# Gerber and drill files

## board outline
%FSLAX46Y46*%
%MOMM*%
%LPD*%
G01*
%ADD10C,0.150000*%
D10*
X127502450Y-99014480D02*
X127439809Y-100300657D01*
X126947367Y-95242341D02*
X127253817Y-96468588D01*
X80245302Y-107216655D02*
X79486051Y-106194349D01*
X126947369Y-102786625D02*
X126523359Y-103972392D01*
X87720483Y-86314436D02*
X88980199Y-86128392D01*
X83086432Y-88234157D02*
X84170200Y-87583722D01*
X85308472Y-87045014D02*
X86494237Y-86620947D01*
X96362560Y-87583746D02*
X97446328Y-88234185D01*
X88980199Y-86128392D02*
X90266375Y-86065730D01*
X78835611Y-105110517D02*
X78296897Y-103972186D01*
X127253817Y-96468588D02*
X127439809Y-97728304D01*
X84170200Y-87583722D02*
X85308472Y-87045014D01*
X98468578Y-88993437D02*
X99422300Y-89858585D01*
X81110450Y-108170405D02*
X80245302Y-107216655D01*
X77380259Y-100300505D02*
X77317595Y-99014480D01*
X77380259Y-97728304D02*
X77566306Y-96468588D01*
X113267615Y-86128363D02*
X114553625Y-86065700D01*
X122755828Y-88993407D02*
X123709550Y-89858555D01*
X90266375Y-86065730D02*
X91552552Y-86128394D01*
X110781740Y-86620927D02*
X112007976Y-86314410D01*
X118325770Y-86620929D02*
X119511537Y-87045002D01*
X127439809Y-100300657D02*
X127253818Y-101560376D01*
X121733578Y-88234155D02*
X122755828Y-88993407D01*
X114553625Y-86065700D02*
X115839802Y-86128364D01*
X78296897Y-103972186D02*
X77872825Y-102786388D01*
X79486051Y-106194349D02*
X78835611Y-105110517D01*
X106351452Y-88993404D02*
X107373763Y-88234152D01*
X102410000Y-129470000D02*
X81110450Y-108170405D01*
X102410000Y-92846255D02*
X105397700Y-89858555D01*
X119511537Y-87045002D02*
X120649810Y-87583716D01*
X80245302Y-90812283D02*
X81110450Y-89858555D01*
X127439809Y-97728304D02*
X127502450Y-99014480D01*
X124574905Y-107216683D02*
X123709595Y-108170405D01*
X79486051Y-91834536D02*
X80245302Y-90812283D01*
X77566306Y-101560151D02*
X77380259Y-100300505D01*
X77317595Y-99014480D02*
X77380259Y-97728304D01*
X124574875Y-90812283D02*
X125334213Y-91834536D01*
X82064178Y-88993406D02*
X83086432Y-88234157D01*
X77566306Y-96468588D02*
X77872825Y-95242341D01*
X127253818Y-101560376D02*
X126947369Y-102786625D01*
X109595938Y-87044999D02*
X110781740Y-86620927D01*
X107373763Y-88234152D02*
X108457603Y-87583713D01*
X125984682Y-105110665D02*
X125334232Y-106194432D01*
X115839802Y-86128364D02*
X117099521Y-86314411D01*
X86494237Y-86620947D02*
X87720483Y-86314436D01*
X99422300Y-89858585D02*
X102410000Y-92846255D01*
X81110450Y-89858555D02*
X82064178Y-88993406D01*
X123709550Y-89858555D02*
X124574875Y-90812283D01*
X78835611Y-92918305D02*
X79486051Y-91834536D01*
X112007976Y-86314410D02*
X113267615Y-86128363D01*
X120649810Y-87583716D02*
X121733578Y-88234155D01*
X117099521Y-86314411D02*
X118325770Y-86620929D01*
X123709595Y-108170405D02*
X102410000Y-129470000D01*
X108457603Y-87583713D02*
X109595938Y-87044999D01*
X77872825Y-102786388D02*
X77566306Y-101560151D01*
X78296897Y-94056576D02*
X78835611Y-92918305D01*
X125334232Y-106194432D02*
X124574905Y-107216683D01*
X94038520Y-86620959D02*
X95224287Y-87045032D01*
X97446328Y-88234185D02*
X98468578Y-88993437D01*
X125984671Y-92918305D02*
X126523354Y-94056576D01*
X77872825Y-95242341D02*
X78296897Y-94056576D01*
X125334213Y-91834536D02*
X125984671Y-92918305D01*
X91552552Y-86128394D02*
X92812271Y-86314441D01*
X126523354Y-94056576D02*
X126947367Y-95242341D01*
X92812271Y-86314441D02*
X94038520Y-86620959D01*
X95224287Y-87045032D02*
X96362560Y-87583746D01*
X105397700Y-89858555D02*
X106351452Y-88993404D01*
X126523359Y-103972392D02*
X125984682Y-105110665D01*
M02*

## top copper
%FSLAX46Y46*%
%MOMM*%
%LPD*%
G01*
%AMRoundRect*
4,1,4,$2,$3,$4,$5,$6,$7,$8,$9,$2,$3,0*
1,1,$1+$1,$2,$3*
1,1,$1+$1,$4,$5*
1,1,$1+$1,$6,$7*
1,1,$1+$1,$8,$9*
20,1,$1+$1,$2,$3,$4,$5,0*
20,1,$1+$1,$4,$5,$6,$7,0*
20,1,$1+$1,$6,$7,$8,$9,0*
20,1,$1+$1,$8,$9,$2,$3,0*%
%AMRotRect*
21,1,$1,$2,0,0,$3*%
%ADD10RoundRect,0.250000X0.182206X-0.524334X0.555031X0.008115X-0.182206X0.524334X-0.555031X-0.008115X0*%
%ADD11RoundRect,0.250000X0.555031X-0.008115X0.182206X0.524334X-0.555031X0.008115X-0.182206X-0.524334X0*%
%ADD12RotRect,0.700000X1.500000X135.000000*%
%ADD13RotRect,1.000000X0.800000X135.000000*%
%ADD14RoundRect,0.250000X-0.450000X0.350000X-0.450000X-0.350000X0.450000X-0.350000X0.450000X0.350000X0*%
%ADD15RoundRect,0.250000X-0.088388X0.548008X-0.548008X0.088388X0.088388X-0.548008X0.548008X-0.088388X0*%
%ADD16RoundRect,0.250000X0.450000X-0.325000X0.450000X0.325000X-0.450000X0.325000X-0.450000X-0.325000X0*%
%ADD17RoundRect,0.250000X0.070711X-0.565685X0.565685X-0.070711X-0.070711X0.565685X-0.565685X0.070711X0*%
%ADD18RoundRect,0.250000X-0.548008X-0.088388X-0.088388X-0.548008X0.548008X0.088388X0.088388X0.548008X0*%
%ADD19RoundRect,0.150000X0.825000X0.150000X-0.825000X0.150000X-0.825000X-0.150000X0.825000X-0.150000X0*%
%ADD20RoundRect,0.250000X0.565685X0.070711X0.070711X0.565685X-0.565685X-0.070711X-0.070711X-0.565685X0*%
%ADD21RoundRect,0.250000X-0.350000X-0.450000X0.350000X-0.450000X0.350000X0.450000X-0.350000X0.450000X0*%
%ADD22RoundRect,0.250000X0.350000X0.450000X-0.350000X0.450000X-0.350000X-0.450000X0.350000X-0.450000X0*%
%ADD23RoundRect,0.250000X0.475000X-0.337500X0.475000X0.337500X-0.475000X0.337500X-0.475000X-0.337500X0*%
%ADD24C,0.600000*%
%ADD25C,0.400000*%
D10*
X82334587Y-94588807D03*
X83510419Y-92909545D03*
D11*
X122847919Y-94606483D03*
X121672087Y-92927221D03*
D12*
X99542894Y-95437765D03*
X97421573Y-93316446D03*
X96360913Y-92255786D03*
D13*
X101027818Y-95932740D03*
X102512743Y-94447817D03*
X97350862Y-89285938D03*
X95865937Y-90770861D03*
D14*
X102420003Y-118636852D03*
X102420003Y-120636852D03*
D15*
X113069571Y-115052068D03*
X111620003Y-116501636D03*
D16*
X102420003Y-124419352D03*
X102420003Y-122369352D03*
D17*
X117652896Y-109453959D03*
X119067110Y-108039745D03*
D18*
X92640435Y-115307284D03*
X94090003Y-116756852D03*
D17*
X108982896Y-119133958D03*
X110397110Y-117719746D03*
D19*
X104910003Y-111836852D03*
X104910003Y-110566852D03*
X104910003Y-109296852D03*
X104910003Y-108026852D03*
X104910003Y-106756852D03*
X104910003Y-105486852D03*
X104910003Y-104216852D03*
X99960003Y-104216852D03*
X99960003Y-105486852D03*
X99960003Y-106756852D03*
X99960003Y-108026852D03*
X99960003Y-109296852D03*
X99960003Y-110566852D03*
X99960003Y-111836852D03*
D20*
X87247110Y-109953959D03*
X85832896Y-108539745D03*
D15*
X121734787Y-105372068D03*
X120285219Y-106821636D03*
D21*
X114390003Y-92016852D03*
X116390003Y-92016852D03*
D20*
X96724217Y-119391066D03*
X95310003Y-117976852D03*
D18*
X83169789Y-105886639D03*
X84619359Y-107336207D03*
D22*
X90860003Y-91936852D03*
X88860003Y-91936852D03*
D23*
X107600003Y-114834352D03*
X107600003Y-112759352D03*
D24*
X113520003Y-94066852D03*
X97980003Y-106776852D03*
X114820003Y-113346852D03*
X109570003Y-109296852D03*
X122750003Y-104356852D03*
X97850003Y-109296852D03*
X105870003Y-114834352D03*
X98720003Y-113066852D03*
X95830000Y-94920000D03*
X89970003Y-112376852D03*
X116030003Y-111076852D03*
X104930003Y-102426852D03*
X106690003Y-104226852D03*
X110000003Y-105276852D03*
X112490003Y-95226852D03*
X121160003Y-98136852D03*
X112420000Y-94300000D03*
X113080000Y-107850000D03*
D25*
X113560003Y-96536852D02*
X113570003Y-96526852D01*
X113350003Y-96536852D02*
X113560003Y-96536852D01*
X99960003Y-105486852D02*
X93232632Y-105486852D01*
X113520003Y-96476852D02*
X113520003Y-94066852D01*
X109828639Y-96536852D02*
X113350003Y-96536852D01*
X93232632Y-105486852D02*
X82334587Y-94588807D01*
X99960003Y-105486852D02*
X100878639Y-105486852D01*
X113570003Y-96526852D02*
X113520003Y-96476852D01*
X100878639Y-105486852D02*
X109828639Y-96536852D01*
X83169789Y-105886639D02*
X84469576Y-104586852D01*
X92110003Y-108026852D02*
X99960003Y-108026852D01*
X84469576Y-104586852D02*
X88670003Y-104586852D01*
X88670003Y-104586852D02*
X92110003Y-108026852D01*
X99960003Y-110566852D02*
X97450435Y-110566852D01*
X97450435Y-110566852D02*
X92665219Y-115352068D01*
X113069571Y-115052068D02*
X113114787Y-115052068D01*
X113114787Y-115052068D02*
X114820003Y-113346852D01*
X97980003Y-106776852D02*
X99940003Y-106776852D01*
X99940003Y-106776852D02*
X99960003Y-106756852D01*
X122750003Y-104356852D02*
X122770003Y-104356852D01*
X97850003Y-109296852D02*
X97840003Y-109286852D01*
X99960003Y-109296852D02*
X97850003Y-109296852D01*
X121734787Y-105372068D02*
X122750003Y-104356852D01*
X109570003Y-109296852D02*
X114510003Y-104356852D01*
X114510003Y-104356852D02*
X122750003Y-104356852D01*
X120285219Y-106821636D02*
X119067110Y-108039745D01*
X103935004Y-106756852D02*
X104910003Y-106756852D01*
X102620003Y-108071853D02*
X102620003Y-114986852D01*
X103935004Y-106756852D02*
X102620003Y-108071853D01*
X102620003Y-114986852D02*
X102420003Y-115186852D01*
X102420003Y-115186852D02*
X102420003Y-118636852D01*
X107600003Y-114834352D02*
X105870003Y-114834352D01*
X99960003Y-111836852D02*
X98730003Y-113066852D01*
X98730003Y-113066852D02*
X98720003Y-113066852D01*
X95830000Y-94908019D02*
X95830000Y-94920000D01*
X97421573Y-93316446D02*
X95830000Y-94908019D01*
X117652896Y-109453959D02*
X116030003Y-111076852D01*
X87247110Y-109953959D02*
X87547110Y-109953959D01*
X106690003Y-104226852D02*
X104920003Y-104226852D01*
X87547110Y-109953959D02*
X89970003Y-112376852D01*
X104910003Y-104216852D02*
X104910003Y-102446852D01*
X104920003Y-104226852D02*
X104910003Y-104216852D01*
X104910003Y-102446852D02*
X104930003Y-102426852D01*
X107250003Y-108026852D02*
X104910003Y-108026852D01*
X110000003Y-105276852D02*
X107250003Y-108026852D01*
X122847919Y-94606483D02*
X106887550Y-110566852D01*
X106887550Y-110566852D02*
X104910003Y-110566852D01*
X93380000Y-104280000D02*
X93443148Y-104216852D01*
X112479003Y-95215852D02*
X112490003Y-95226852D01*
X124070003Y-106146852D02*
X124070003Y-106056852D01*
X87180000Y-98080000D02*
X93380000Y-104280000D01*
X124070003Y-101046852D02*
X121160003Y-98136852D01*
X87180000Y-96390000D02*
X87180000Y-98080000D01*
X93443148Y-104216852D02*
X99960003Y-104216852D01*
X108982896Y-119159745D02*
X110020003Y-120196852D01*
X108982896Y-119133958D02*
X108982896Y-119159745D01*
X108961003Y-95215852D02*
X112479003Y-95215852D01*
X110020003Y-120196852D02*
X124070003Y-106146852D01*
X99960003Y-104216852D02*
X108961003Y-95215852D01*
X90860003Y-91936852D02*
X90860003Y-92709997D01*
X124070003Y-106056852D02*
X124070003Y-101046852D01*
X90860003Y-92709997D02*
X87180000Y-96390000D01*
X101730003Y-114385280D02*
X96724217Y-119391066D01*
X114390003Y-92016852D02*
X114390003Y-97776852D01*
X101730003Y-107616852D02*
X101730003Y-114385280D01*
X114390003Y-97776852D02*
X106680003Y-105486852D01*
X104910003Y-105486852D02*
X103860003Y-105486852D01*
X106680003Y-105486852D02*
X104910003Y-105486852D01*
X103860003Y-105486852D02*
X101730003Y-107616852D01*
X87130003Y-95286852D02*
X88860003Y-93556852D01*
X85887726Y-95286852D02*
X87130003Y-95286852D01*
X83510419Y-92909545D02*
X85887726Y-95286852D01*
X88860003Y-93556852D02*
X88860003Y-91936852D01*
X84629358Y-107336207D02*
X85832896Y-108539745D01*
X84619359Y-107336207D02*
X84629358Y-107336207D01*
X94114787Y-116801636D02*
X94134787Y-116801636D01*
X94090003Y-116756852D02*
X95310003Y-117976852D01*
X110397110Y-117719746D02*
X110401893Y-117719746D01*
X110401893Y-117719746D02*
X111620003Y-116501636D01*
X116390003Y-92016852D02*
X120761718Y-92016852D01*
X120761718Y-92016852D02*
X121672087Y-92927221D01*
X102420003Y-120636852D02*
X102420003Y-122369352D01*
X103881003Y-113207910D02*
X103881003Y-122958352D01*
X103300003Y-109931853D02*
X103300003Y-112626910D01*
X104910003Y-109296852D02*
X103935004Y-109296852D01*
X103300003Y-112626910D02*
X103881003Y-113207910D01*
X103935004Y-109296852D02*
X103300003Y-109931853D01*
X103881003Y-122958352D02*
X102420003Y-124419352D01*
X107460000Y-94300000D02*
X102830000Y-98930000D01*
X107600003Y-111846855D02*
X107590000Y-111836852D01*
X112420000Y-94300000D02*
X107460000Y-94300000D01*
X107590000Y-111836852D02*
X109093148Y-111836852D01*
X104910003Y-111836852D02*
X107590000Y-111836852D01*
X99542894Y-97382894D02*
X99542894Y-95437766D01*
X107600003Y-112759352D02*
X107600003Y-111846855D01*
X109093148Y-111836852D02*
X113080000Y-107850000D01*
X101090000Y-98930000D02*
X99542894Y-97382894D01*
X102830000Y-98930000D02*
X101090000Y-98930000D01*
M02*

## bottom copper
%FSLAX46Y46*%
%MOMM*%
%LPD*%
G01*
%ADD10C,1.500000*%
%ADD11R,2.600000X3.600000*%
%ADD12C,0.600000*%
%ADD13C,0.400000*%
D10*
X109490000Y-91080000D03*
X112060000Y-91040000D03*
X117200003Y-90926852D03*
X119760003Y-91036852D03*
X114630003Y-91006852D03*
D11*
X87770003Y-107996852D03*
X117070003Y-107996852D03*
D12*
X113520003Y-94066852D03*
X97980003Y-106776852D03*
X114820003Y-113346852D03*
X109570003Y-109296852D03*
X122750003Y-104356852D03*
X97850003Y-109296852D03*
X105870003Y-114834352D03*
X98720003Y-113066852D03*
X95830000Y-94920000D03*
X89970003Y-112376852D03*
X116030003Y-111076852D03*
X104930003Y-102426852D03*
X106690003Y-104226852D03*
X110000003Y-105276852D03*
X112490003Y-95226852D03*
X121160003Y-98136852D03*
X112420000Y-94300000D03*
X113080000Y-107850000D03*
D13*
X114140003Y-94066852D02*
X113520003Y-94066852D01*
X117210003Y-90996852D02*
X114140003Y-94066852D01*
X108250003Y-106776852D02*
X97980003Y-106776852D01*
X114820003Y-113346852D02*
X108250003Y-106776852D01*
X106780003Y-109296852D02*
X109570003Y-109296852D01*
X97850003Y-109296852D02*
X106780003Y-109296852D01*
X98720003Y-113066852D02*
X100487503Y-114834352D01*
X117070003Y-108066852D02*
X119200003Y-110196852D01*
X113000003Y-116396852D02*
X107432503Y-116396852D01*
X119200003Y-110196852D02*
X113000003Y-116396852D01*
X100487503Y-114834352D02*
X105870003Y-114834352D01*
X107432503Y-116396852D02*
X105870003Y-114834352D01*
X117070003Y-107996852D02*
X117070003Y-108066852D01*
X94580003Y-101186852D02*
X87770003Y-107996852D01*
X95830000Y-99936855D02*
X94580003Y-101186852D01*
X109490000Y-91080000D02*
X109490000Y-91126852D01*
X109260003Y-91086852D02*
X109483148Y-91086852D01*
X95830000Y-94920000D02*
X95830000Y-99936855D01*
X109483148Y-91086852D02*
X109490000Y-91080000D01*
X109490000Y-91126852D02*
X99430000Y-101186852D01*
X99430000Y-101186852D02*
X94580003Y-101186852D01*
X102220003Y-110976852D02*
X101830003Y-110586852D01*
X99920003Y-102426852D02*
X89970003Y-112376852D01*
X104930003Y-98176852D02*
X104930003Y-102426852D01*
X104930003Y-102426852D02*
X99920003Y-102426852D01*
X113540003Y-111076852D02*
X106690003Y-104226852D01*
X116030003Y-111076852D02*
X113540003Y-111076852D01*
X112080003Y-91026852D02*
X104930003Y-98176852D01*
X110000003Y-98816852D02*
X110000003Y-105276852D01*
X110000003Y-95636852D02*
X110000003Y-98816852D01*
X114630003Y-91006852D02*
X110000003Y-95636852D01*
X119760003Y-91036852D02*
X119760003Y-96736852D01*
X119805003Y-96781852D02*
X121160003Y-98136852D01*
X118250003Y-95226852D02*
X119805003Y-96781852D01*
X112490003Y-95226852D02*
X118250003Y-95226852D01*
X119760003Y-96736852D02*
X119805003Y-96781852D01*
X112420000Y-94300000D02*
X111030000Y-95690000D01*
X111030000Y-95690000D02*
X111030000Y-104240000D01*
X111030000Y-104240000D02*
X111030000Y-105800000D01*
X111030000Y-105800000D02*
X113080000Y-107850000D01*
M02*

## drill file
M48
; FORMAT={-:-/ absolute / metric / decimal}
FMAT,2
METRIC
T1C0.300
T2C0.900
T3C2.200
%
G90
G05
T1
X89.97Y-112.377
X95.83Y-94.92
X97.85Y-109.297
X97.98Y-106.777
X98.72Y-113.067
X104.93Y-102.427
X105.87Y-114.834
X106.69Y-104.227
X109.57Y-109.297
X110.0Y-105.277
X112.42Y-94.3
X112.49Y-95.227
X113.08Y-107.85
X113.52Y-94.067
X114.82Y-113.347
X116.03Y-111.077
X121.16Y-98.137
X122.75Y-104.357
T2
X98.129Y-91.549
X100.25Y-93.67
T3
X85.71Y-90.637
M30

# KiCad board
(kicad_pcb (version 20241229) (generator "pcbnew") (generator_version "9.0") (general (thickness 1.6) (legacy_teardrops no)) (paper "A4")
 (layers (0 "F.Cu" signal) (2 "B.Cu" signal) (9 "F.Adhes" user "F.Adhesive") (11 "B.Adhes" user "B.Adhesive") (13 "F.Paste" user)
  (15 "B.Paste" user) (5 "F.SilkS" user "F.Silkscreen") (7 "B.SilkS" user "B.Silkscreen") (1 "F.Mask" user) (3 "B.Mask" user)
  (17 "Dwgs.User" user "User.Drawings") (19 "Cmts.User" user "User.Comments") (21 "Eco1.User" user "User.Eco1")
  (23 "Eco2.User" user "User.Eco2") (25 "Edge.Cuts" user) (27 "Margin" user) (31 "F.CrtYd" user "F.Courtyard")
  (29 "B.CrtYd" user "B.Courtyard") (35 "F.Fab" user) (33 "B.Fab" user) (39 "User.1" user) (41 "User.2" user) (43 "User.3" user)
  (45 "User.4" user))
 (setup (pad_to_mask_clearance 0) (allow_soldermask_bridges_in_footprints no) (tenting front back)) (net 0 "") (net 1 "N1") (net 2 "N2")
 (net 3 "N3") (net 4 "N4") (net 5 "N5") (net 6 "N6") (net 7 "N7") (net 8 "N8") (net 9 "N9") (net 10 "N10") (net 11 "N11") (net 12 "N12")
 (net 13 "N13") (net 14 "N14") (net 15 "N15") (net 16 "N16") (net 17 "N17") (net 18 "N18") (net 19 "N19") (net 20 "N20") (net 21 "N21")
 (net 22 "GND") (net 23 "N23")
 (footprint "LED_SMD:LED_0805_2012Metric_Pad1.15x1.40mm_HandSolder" (layer "F.Cu") (at 82.922503 93.749176 55)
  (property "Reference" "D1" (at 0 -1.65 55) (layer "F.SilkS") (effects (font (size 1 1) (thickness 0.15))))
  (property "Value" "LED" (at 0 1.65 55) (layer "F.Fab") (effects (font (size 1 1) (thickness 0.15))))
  (pad "1" smd roundrect (at -1.025 0 55) (size 1.15 1.4) (layers "F.Cu" "F.Mask" "F.Paste") (roundrect_rratio 0.217391) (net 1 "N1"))
  (pad "2" smd roundrect (at 1.025 0 55) (size 1.15 1.4) (layers "F.Cu" "F.Mask" "F.Paste") (roundrect_rratio 0.217391) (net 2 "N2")))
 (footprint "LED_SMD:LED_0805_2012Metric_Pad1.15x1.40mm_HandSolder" (layer "F.Cu") (at 122.260003 93.766852 125)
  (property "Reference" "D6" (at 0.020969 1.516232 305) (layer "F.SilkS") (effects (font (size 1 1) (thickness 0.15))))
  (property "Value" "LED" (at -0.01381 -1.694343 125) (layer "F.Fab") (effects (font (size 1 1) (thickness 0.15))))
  (pad "1" smd roundrect (at -1.025 0 125) (size 1.15 1.4) (layers "F.Cu" "F.Mask" "F.Paste") (roundrect_rratio 0.217391) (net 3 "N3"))
  (pad "2" smd roundrect (at 1.025 0 125) (size 1.15 1.4) (layers "F.Cu" "F.Mask" "F.Paste") (roundrect_rratio 0.217391) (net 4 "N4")))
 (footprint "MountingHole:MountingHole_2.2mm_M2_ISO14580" (layer "F.Cu") (at 85.710003 90.636852)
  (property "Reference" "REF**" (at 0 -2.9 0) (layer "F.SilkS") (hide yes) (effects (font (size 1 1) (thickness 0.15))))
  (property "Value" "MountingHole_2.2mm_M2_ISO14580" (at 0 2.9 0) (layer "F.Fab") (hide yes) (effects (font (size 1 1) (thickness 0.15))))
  (pad "" np_thru_hole circle (at 0 0) (size 2.2 2.2) (drill 2.2) (layers "*.Cu" "*.Mask")))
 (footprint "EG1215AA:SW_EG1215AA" (layer "F.Cu") (at 99.18934 92.609339 135)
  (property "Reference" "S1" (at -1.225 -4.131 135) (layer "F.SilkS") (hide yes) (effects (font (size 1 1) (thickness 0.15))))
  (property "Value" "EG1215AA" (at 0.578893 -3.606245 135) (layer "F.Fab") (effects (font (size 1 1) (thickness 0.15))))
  (pad "" np_thru_hole circle (at -1.5 -0.000001 135) (size 0.9 0.9) (drill 0.9) (layers "*.Cu" "*.Mask"))
  (pad "" np_thru_hole circle (at 1.5 0.000001 135) (size 0.9 0.9) (drill 0.9) (layers "*.Cu" "*.Mask"))
  (pad "1" smd rect (at -2.25 -1.749999 135) (size 0.7 1.5) (layers "F.Cu" "F.Mask" "F.Paste") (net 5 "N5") (solder_mask_margin 0.102))
  (pad "2" smd rect (at 0.75 -1.75 135) (size 0.7 1.5) (layers "F.Cu" "F.Mask" "F.Paste") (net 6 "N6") (solder_mask_margin 0.102))
  (pad "3" smd rect (at 2.25 -1.75 135) (size 0.7 1.5) (layers "F.Cu" "F.Mask" "F.Paste") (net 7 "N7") (solder_mask_margin 0.102))
  (pad "S1" smd rect (at -3.65 -1.049999 135) (size 1 0.8) (layers "F.Cu" "F.Mask" "F.Paste") (solder_mask_margin 0.102))
  (pad "S2" smd rect (at -3.650001 1.050001 135) (size 1 0.8) (layers "F.Cu" "F.Mask" "F.Paste") (solder_mask_margin 0.102))
  (pad "S3" smd rect (at 3.65 1.049999 135) (size 1 0.8) (layers "F.Cu" "F.Mask" "F.Paste") (solder_mask_margin 0.102))
  (pad "S4" smd rect (at 3.650001 -1.050001 135) (size 1 0.8) (layers "F.Cu" "F.Mask" "F.Paste") (solder_mask_margin 0.102)))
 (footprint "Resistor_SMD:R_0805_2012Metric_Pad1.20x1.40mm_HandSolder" (layer "F.Cu") (at 102.420003 119.636852 -90)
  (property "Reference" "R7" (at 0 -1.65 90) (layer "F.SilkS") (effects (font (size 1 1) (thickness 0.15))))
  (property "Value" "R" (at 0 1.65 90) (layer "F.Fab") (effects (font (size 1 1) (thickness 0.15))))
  (pad "1" smd roundrect (at -1 0 270) (size 1.2 1.4) (layers "F.Cu" "F.Mask" "F.Paste") (roundrect_rratio 0.208333) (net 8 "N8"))
  (pad "2" smd roundrect (at 1 0 270) (size 1.2 1.4) (layers "F.Cu" "F.Mask" "F.Paste") (roundrect_rratio 0.208333) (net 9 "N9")))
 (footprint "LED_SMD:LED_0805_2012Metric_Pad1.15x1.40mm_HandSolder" (layer "F.Cu") (at 112.344787 115.776852 -135)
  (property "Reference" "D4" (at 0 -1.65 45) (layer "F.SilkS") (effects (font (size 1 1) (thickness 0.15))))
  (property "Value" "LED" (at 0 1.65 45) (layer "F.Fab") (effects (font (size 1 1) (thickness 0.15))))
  (pad "1" smd roundrect (at -1.024999 0 225) (size 1.15 1.4) (layers "F.Cu" "F.Mask" "F.Paste") (roundrect_rratio 0.217391) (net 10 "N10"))
  (pad "2" smd roundrect (at 1.024999 0 225) (size 1.15 1.4) (layers "F.Cu" "F.Mask" "F.Paste") (roundrect_rratio 0.217391) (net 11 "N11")))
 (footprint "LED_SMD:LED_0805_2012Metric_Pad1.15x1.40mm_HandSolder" (layer "F.Cu") (at 102.420003 123.394352 90)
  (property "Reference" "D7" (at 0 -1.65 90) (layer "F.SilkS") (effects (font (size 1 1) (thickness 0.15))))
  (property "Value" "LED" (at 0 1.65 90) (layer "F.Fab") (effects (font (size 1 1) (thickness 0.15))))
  (pad "1" smd roundrect (at -1.025 0 90) (size 1.15 1.4) (layers "F.Cu" "F.Mask" "F.Paste") (roundrect_rratio 0.217391) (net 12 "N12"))
  (pad "2" smd roundrect (at 1.025 0 90) (size 1.15 1.4) (layers "F.Cu" "F.Mask" "F.Paste") (roundrect_rratio 0.217391) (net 9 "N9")))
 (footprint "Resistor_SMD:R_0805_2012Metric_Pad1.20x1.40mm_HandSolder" (layer "F.Cu") (at 118.360003 108.746852 45)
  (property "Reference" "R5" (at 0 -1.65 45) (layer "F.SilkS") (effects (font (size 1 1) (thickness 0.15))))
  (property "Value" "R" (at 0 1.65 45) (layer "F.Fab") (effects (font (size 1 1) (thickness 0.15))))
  (pad "1" smd roundrect (at -1 0 45) (size 1.2 1.4) (layers "F.Cu" "F.Mask" "F.Paste") (roundrect_rratio 0.208333) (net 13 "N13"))
  (pad "2" smd roundrect (at 1 0 45) (size 1.2 1.4) (layers "F.Cu" "F.Mask" "F.Paste") (roundrect_rratio 0.208333) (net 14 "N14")))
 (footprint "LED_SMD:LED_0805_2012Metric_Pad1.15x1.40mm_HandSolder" (layer "F.Cu") (at 93.365219 116.032068 -45)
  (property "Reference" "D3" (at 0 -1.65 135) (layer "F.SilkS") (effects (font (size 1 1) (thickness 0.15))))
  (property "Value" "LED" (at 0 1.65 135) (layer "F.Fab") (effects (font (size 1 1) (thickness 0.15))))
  (pad "1" smd roundrect (at -1.024999 0 315) (size 1.15 1.4) (layers "F.Cu" "F.Mask" "F.Paste") (roundrect_rratio 0.217391) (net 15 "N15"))
  (pad "2" smd roundrect (at 1.024999 0 315) (size 1.15 1.4) (layers "F.Cu" "F.Mask" "F.Paste") (roundrect_rratio 0.217391) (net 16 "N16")))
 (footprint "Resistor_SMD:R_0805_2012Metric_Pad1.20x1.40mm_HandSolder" (layer "F.Cu") (at 109.690003 118.426852 45)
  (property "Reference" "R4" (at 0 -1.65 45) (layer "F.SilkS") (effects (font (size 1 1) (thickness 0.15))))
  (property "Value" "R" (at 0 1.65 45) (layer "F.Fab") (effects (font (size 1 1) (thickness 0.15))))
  (pad "1" smd roundrect (at -1 -0.000001 45) (size 1.2 1.4) (layers "F.Cu" "F.Mask" "F.Paste") (roundrect_rratio 0.208333) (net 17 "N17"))
  (pad "2" smd roundrect (at 1 0.000001 45) (size 1.2 1.4) (layers "F.Cu" "F.Mask" "F.Paste") (roundrect_rratio 0.208333) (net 11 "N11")))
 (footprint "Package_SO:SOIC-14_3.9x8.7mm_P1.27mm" (layer "F.Cu") (at 102.435003 108.026852 180)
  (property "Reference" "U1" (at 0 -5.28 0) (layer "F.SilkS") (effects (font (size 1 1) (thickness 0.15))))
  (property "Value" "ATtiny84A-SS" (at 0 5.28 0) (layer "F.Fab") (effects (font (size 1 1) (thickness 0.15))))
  (pad "1" smd roundrect (at -2.475 -3.81 180) (size 1.95 0.6) (layers "F.Cu" "F.Mask" "F.Paste") (roundrect_rratio 0.25) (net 5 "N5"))
  (pad "2" smd roundrect (at -2.475 -2.54 180) (size 1.95 0.6) (layers "F.Cu" "F.Mask" "F.Paste") (roundrect_rratio 0.25) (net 3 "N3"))
  (pad "3" smd roundrect (at -2.475 -1.27 180) (size 1.95 0.6) (layers "F.Cu" "F.Mask" "F.Paste") (roundrect_rratio 0.25) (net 12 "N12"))
  (pad "4" smd roundrect (at -2.475 0 180) (size 1.95 0.6) (layers "F.Cu" "F.Mask" "F.Paste") (roundrect_rratio 0.25) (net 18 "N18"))
  (pad "5" smd roundrect (at -2.475 1.27 180) (size 1.95 0.6) (layers "F.Cu" "F.Mask" "F.Paste") (roundrect_rratio 0.25) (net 8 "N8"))
  (pad "6" smd roundrect (at -2.475 2.54 180) (size 1.95 0.6) (layers "F.Cu" "F.Mask" "F.Paste") (roundrect_rratio 0.25) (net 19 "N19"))
  (pad "7" smd roundrect (at -2.475 3.81 180) (size 1.95 0.6) (layers "F.Cu" "F.Mask" "F.Paste") (roundrect_rratio 0.25) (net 13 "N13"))
  (pad "8" smd roundrect (at 2.475 3.81 180) (size 1.95 0.6) (layers "F.Cu" "F.Mask" "F.Paste") (roundrect_rratio 0.25) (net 17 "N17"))
  (pad "9" smd roundrect (at 2.475 2.54 180) (size 1.95 0.6) (layers "F.Cu" "F.Mask" "F.Paste") (roundrect_rratio 0.25) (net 1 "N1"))
  (pad "10" smd roundrect (at 2.475 1.27 180) (size 1.95 0.6) (layers "F.Cu" "F.Mask" "F.Paste") (roundrect_rratio 0.25) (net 10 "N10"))
  (pad "11" smd roundrect (at 2.475 0 180) (size 1.95 0.6) (layers "F.Cu" "F.Mask" "F.Paste") (roundrect_rratio 0.25) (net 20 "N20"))
  (pad "12" smd roundrect (at 2.475 -1.27 180) (size 1.95 0.6) (layers "F.Cu" "F.Mask" "F.Paste") (roundrect_rratio 0.25) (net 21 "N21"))
  (pad "13" smd roundrect (at 2.475 -2.54 180) (size 1.95 0.6) (layers "F.Cu" "F.Mask" "F.Paste") (roundrect_rratio 0.25) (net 15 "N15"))
  (pad "14" smd roundrect (at 2.475 -3.81 180) (size 1.95 0.6) (layers "F.Cu" "F.Mask" "F.Paste") (roundrect_rratio 0.25) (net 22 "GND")))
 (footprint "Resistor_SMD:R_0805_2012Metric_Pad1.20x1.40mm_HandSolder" (layer "F.Cu") (at 86.540003 109.246852 135)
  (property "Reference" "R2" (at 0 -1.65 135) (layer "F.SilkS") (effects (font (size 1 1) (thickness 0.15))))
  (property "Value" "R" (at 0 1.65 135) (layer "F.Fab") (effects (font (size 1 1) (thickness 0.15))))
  (pad "1" smd roundrect (at -1 0 135) (size 1.2 1.4) (layers "F.Cu" "F.Mask" "F.Paste") (roundrect_rratio 0.208333) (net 13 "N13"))
  (pad "2" smd roundrect (at 1 0 135) (size 1.2 1.4) (layers "F.Cu" "F.Mask" "F.Paste") (roundrect_rratio 0.208333) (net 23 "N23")))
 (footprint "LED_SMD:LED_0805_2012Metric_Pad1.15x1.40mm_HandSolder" (layer "F.Cu") (at 121.010003 106.096852 -135)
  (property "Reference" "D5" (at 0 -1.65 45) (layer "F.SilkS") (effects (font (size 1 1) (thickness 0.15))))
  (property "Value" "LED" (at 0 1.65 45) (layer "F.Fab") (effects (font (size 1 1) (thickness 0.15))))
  (pad "1" smd roundrect (at -1.024999 0 225) (size 1.15 1.4) (layers "F.Cu" "F.Mask" "F.Paste") (roundrect_rratio 0.217391) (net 21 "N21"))
  (pad "2" smd roundrect (at 1.024999 0 225) (size 1.15 1.4) (layers "F.Cu" "F.Mask" "F.Paste") (roundrect_rratio 0.217391) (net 14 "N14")))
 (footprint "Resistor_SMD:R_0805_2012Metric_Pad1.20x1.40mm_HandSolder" (layer "F.Cu") (at 115.390003 92.016852)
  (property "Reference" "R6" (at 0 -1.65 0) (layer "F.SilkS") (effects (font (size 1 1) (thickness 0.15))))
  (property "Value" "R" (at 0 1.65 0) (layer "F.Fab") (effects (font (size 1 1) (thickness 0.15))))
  (pad "1" smd roundrect (at -1 0) (size 1.2 1.4) (layers "F.Cu" "F.Mask" "F.Paste") (roundrect_rratio 0.208333) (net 19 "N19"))
  (pad "2" smd roundrect (at 1 0) (size 1.2 1.4) (layers "F.Cu" "F.Mask" "F.Paste") (roundrect_rratio 0.208333) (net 4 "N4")))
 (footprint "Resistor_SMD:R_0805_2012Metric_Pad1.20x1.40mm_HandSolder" (layer "F.Cu") (at 96.01711 118.683959 135)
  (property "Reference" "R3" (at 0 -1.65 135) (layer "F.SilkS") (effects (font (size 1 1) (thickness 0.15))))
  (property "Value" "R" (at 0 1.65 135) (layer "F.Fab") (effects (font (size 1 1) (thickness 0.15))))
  (pad "1" smd roundrect (at -1 0 135) (size 1.2 1.4) (layers "F.Cu" "F.Mask" "F.Paste") (roundrect_rratio 0.208333) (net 19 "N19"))
  (pad "2" smd roundrect (at 1 0 135) (size 1.2 1.4) (layers "F.Cu" "F.Mask" "F.Paste") (roundrect_rratio 0.208333) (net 16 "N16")))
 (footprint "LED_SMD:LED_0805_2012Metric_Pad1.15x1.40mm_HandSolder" (layer "F.Cu") (at 83.894574 106.611423 -45)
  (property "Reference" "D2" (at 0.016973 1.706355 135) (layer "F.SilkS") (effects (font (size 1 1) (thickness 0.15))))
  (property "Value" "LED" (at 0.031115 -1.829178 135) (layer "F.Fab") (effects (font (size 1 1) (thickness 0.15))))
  (pad "1" smd roundrect (at -1.025 0.000001 315) (size 1.15 1.4) (layers "F.Cu" "F.Mask" "F.Paste") (roundrect_rratio 0.217391)
   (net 20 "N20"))
  (pad "2" smd roundrect (at 1.025 -0.000001 315) (size 1.15 1.4) (layers "F.Cu" "F.Mask" "F.Paste") (roundrect_rratio 0.217391)
   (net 23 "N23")))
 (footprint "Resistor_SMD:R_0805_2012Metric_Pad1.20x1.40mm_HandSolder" (layer "F.Cu") (at 89.860003 91.936852 180)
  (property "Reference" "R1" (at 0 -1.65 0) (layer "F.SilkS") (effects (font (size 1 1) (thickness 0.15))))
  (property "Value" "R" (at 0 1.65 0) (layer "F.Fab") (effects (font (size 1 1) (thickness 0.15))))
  (pad "1" smd roundrect (at -1 0 180) (size 1.2 1.4) (layers "F.Cu" "F.Mask" "F.Paste") (roundrect_rratio 0.208333) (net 17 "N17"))
  (pad "2" smd roundrect (at 1 0 180) (size 1.2 1.4) (layers "F.Cu" "F.Mask" "F.Paste") (roundrect_rratio 0.208333) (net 2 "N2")))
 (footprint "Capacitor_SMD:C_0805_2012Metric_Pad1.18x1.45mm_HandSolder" (layer "F.Cu") (at 107.600003 113.796852 90)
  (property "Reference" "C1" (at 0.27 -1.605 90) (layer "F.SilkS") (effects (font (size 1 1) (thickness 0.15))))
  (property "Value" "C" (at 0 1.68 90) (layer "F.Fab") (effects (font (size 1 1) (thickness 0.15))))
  (pad "1" smd roundrect (at -1.0375 0 90) (size 1.175 1.45) (layers "F.Cu" "F.Mask" "F.Paste") (roundrect_rratio 0.212766) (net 22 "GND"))
  (pad "2" smd roundrect (at 1.0375 0 90) (size 1.175 1.45) (layers "F.Cu" "F.Mask" "F.Paste") (roundrect_rratio 0.212766) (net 5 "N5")))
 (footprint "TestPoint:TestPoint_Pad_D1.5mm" (layer "B.Cu") (at 109.49 91.08)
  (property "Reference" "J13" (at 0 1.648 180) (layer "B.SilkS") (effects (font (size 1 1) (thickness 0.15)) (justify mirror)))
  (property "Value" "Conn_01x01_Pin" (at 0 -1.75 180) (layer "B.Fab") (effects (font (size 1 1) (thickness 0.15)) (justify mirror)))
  (pad "1" smd circle (at 0 0) (size 1.5 1.5) (layers "B.Cu" "B.Mask") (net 6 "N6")))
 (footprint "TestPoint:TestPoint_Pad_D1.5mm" (layer "B.Cu") (at 112.06 91.04)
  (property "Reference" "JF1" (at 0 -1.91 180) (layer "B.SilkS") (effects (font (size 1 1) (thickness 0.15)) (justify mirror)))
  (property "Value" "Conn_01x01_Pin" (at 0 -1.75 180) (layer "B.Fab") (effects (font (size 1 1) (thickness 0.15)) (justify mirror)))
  (pad "1" smd circle (at 0 0) (size 1.5 1.5) (layers "B.Cu" "B.Mask") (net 13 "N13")))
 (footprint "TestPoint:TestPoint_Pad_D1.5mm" (layer "B.Cu") (at 117.200003 90.926852)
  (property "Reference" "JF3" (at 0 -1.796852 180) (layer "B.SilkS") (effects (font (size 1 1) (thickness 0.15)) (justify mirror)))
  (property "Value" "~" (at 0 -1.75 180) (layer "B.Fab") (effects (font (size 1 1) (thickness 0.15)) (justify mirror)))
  (pad "1" smd circle (at 0 0) (size 1.5 1.5) (layers "B.Cu" "B.Mask") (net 1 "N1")))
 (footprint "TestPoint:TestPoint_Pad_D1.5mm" (layer "B.Cu") (at 119.760003 91.036852)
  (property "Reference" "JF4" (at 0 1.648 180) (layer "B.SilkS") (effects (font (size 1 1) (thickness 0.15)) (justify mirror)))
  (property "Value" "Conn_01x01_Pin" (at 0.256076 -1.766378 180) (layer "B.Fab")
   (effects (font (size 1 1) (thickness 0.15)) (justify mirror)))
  (pad "1" smd circle (at 0 0) (size 1.5 1.5) (layers "B.Cu" "B.Mask") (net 17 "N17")))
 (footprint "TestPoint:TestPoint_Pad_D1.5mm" (layer "B.Cu") (at 114.630003 91.006852)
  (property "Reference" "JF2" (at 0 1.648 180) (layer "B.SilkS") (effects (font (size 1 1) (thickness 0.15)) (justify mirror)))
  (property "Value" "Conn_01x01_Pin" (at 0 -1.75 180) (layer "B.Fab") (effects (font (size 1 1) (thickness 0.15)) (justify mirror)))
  (pad "1" smd circle (at 0 0) (size 1.5 1.5) (layers "B.Cu" "B.Mask") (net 18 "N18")))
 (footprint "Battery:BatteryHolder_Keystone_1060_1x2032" (layer "B.Cu") (at 102.420003 107.996852)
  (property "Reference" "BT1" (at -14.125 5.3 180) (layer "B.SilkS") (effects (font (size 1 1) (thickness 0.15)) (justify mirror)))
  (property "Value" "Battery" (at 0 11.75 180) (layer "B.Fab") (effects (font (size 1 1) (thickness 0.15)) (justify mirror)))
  (pad "1" smd rect (at -14.65 0 180) (size 2.6 3.6) (layers "B.Cu" "B.Mask" "B.Paste") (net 6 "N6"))
  (pad "2" smd rect (at 14.65 0 180) (size 2.6 3.6) (layers "B.Cu" "B.Mask" "B.Paste") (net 22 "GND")))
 (gr_line (start 127.50245 99.01448) (end 127.439809 100.300657) (stroke (width 0.15) (type default)) (layer "Edge.Cuts"))
 (gr_line (start 126.947367 95.242341) (end 127.253817 96.468588) (stroke (width 0.15) (type default)) (layer "Edge.Cuts"))
 (gr_line (start 80.245302 107.216655) (end 79.486051 106.194349) (stroke (width 0.15) (type default)) (layer "Edge.Cuts"))
 (gr_line (start 126.947369 102.786625) (end 126.523359 103.972392) (stroke (width 0.15) (type default)) (layer "Edge.Cuts"))
 (gr_line (start 87.720483 86.314436) (end 88.980199 86.128392) (stroke (width 0.15) (type default)) (layer "Edge.Cuts"))
 (gr_line (start 83.086432 88.234157) (end 84.1702 87.583722) (stroke (width 0.15) (type default)) (layer "Edge.Cuts"))
 (gr_line (start 85.308472 87.045014) (end 86.494237 86.620947) (stroke (width 0.15) (type default)) (layer "Edge.Cuts"))
 (gr_line (start 96.36256 87.583746) (end 97.446328 88.234185) (stroke (width 0.15) (type default)) (layer "Edge.Cuts"))
 (gr_line (start 88.980199 86.128392) (end 90.266375 86.06573) (stroke (width 0.15) (type default)) (layer "Edge.Cuts"))
 (gr_line (start 78.835611 105.110517) (end 78.296897 103.972186) (stroke (width 0.15) (type default)) (layer "Edge.Cuts"))
 (gr_line (start 127.253817 96.468588) (end 127.439809 97.728304) (stroke (width 0.15) (type default)) (layer "Edge.Cuts"))
 (gr_line (start 84.1702 87.583722) (end 85.308472 87.045014) (stroke (width 0.15) (type default)) (layer "Edge.Cuts"))
 (gr_line (start 98.468578 88.993437) (end 99.4223 89.858585) (stroke (width 0.15) (type default)) (layer "Edge.Cuts"))
 (gr_line (start 81.11045 108.170405) (end 80.245302 107.216655) (stroke (width 0.15) (type default)) (layer "Edge.Cuts"))
 (gr_line (start 77.380259 100.300505) (end 77.317595 99.01448) (stroke (width 0.15) (type default)) (layer "Edge.Cuts"))
 (gr_line (start 77.380259 97.728304) (end 77.566306 96.468588) (stroke (width 0.15) (type default)) (layer "Edge.Cuts"))
 (gr_line (start 113.267615 86.128363) (end 114.553625 86.0657) (stroke (width 0.15) (type default)) (layer "Edge.Cuts"))
 (gr_line (start 122.755828 88.993407) (end 123.70955 89.858555) (stroke (width 0.15) (type default)) (layer "Edge.Cuts"))
 (gr_line (start 90.266375 86.06573) (end 91.552552 86.128394) (stroke (width 0.15) (type default)) (layer "Edge.Cuts"))
 (gr_line (start 110.78174 86.620927) (end 112.007976 86.31441) (stroke (width 0.15) (type default)) (layer "Edge.Cuts"))
 (gr_line (start 118.32577 86.620929) (end 119.511537 87.045002) (stroke (width 0.15) (type default)) (layer "Edge.Cuts"))
 (gr_line (start 127.439809 100.300657) (end 127.253818 101.560376) (stroke (width 0.15) (type default)) (layer "Edge.Cuts"))
 (gr_line (start 121.733578 88.234155) (end 122.755828 88.993407) (stroke (width 0.15) (type default)) (layer "Edge.Cuts"))
 (gr_line (start 114.553625 86.0657) (end 115.839802 86.128364) (stroke (width 0.15) (type default)) (layer "Edge.Cuts"))
 (gr_line (start 78.296897 103.972186) (end 77.872825 102.786388) (stroke (width 0.15) (type default)) (layer "Edge.Cuts"))
 (gr_line (start 79.486051 106.194349) (end 78.835611 105.110517) (stroke (width 0.15) (type default)) (layer "Edge.Cuts"))
 (gr_line (start 106.351452 88.993404) (end 107.373763 88.234152) (stroke (width 0.15) (type default)) (layer "Edge.Cuts"))
 (gr_line (start 102.41 129.47) (end 81.11045 108.170405) (stroke (width 0.15) (type default)) (layer "Edge.Cuts"))
 (gr_line (start 102.41 92.846255) (end 105.3977 89.858555) (stroke (width 0.15) (type default)) (layer "Edge.Cuts"))
 (gr_line (start 119.511537 87.045002) (end 120.64981 87.583716) (stroke (width 0.15) (type default)) (layer "Edge.Cuts"))
 (gr_line (start 80.245302 90.812283) (end 81.11045 89.858555) (stroke (width 0.15) (type default)) (layer "Edge.Cuts"))
 (gr_line (start 127.439809 97.728304) (end 127.50245 99.01448) (stroke (width 0.15) (type default)) (layer "Edge.Cuts"))
 (gr_line (start 124.574905 107.216683) (end 123.709595 108.170405) (stroke (width 0.15) (type default)) (layer "Edge.Cuts"))
 (gr_line (start 79.486051 91.834536) (end 80.245302 90.812283) (stroke (width 0.15) (type default)) (layer "Edge.Cuts"))
 (gr_line (start 77.566306 101.560151) (end 77.380259 100.300505) (stroke (width 0.15) (type default)) (layer "Edge.Cuts"))
 (gr_line (start 77.317595 99.01448) (end 77.380259 97.728304) (stroke (width 0.15) (type default)) (layer "Edge.Cuts"))
 (gr_line (start 124.574875 90.812283) (end 125.334213 91.834536) (stroke (width 0.15) (type default)) (layer "Edge.Cuts"))
 (gr_line (start 82.064178 88.993406) (end 83.086432 88.234157) (stroke (width 0.15) (type default)) (layer "Edge.Cuts"))
 (gr_line (start 77.566306 96.468588) (end 77.872825 95.242341) (stroke (width 0.15) (type default)) (layer "Edge.Cuts"))
 (gr_line (start 127.253818 101.560376) (end 126.947369 102.786625) (stroke (width 0.15) (type default)) (layer "Edge.Cuts"))
 (gr_line (start 109.595938 87.044999) (end 110.78174 86.620927) (stroke (width 0.15) (type default)) (layer "Edge.Cuts"))
 (gr_line (start 107.373763 88.234152) (end 108.457603 87.583713) (stroke (width 0.15) (type default)) (layer "Edge.Cuts"))
 (gr_line (start 125.984682 105.110665) (end 125.334232 106.194432) (stroke (width 0.15) (type default)) (layer "Edge.Cuts"))
 (gr_line (start 115.839802 86.128364) (end 117.099521 86.314411) (stroke (width 0.15) (type default)) (layer "Edge.Cuts"))
 (gr_line (start 86.494237 86.620947) (end 87.720483 86.314436) (stroke (width 0.15) (type default)) (layer "Edge.Cuts"))
 (gr_line (start 99.4223 89.858585) (end 102.41 92.846255) (stroke (width 0.15) (type default)) (layer "Edge.Cuts"))
 (gr_line (start 81.11045 89.858555) (end 82.064178 88.993406) (stroke (width 0.15) (type default)) (layer "Edge.Cuts"))
 (gr_line (start 123.70955 89.858555) (end 124.574875 90.812283) (stroke (width 0.15) (type default)) (layer "Edge.Cuts"))
 (gr_line (start 78.835611 92.918305) (end 79.486051 91.834536) (stroke (width 0.15) (type default)) (layer "Edge.Cuts"))
 (gr_line (start 112.007976 86.31441) (end 113.267615 86.128363) (stroke (width 0.15) (type default)) (layer "Edge.Cuts"))
 (gr_line (start 120.64981 87.583716) (end 121.733578 88.234155) (stroke (width 0.15) (type default)) (layer "Edge.Cuts"))
 (gr_line (start 117.099521 86.314411) (end 118.32577 86.620929) (stroke (width 0.15) (type default)) (layer "Edge.Cuts"))
 (gr_line (start 123.709595 108.170405) (end 102.41 129.47) (stroke (width 0.15) (type default)) (layer "Edge.Cuts"))
 (gr_line (start 108.457603 87.583713) (end 109.595938 87.044999) (stroke (width 0.15) (type default)) (layer "Edge.Cuts"))
 (gr_line (start 77.872825 102.786388) (end 77.566306 101.560151) (stroke (width 0.15) (type default)) (layer "Edge.Cuts"))
 (gr_line (start 78.296897 94.056576) (end 78.835611 92.918305) (stroke (width 0.15) (type default)) (layer "Edge.Cuts"))
 (gr_line (start 125.334232 106.194432) (end 124.574905 107.216683) (stroke (width 0.15) (type default)) (layer "Edge.Cuts"))
 (gr_line (start 94.03852 86.620959) (end 95.224287 87.045032) (stroke (width 0.15) (type default)) (layer "Edge.Cuts"))
 (gr_line (start 97.446328 88.234185) (end 98.468578 88.993437) (stroke (width 0.15) (type default)) (layer "Edge.Cuts"))
 (gr_line (start 125.984671 92.918305) (end 126.523354 94.056576) (stroke (width 0.15) (type default)) (layer "Edge.Cuts"))
 (gr_line (start 77.872825 95.242341) (end 78.296897 94.056576) (stroke (width 0.15) (type default)) (layer "Edge.Cuts"))
 (gr_line (start 125.334213 91.834536) (end 125.984671 92.918305) (stroke (width 0.15) (type default)) (layer "Edge.Cuts"))
 (gr_line (start 91.552552 86.128394) (end 92.812271 86.314441) (stroke (width 0.15) (type default)) (layer "Edge.Cuts"))
 (gr_line (start 126.523354 94.056576) (end 126.947367 95.242341) (stroke (width 0.15) (type default)) (layer "Edge.Cuts"))
 (gr_line (start 92.812271 86.314441) (end 94.03852 86.620959) (stroke (width 0.15) (type default)) (layer "Edge.Cuts"))
 (gr_line (start 95.224287 87.045032) (end 96.36256 87.583746) (stroke (width 0.15) (type default)) (layer "Edge.Cuts"))
 (gr_line (start 105.3977 89.858555) (end 106.351452 88.993404) (stroke (width 0.15) (type default)) (layer "Edge.Cuts"))
 (gr_line (start 126.523359 103.972392) (end 125.984682 105.110665) (stroke (width 0.15) (type default)) (layer "Edge.Cuts"))
 (segment (start 113.560003 96.536852) (end 113.570003 96.526852) (width 0.4) (layer "F.Cu") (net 1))
 (segment (start 113.350003 96.536852) (end 113.560003 96.536852) (width 0.4) (layer "F.Cu") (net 1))
 (segment (start 99.960003 105.486852) (end 93.232632 105.486852) (width 0.4) (layer "F.Cu") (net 1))
 (segment (start 113.520003 96.476852) (end 113.520003 94.066852) (width 0.4) (layer "F.Cu") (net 1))
 (segment (start 109.828639 96.536852) (end 113.350003 96.536852) (width 0.4) (layer "F.Cu") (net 1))
 (segment (start 93.232632 105.486852) (end 82.334587 94.588807) (width 0.4) (layer "F.Cu") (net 1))
 (segment (start 99.960003 105.486852) (end 100.878639 105.486852) (width 0.4) (layer "F.Cu") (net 1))
 (segment (start 113.570003 96.526852) (end 113.520003 96.476852) (width 0.4) (layer "F.Cu") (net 1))
 (segment (start 100.878639 105.486852) (end 109.828639 96.536852) (width 0.4) (layer "F.Cu") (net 1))
 (via (at 113.520003 94.066852) (size 0.6) (drill 0.3) (layers "F.Cu" "B.Cu") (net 1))
 (segment (start 114.140003 94.066852) (end 113.520003 94.066852) (width 0.4) (layer "B.Cu") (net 1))
 (segment (start 117.210003 90.996852) (end 114.140003 94.066852) (width 0.4) (layer "B.Cu") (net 1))
 (segment (start 83.169789 105.886639) (end 84.469576 104.586852) (width 0.4) (layer "F.Cu") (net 20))
 (segment (start 92.110003 108.026852) (end 99.960003 108.026852) (width 0.4) (layer "F.Cu") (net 20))
 (segment (start 84.469576 104.586852) (end 88.670003 104.586852) (width 0.4) (layer "F.Cu") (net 20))
 (segment (start 88.670003 104.586852) (end 92.110003 108.026852) (width 0.4) (layer "F.Cu") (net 20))
 (segment (start 99.960003 110.566852) (end 97.450435 110.566852) (width 0.4) (layer "F.Cu") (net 15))
 (segment (start 97.450435 110.566852) (end 92.665219 115.352068) (width 0.4) (layer "F.Cu") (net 15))
 (segment (start 113.069571 115.052068) (end 113.114787 115.052068) (width 0.4) (layer "F.Cu") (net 10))
 (segment (start 113.114787 115.052068) (end 114.820003 113.346852) (width 0.4) (layer "F.Cu") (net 10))
 (segment (start 97.980003 106.776852) (end 99.940003 106.776852) (width 0.4) (layer "F.Cu") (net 10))
 (segment (start 99.940003 106.776852) (end 99.960003 106.756852) (width 0.4) (layer "F.Cu") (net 10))
 (via (at 97.980003 106.776852) (size 0.6) (drill 0.3) (layers "F.Cu" "B.Cu") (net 10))
 (via (at 114.820003 113.346852) (size 0.6) (drill 0.3) (layers "F.Cu" "B.Cu") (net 10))
 (segment (start 108.250003 106.776852) (end 97.980003 106.776852) (width 0.4) (layer "B.Cu") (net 10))
 (segment (start 114.820003 113.346852) (end 108.250003 106.776852) (width 0.4) (layer "B.Cu") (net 10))
 (segment (start 122.750003 104.356852) (end 122.770003 104.356852) (width 0.4) (layer "F.Cu") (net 21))
 (segment (start 97.850003 109.296852) (end 97.840003 109.286852) (width 0.4) (layer "F.Cu") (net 21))
 (segment (start 99.960003 109.296852) (end 97.850003 109.296852) (width 0.4) (layer "F.Cu") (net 21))
 (segment (start 121.734787 105.372068) (end 122.750003 104.356852) (width 0.4) (layer "F.Cu") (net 21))
 (segment (start 109.570003 109.296852) (end 114.510003 104.356852) (width 0.4) (layer "F.Cu") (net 21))
 (segment (start 114.510003 104.356852) (end 122.750003 104.356852) (width 0.4) (layer "F.Cu") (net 21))
 (via (at 109.570003 109.296852) (size 0.6) (drill 0.3) (layers "F.Cu" "B.Cu") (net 21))
 (via (at 122.750003 104.356852) (size 0.6) (drill 0.3) (layers "F.Cu" "B.Cu") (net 21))
 (via (at 97.850003 109.296852) (size 0.6) (drill 0.3) (layers "F.Cu" "B.Cu") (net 21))
 (segment (start 106.780003 109.296852) (end 109.570003 109.296852) (width 0.4) (layer "B.Cu") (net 21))
 (segment (start 97.850003 109.296852) (end 106.780003 109.296852) (width 0.4) (layer "B.Cu") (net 21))
 (segment (start 120.285219 106.821636) (end 119.06711 108.039745) (width 0.4) (layer "F.Cu") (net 14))
 (segment (start 103.935004 106.756852) (end 104.910003 106.756852) (width 0.4) (layer "F.Cu") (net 8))
 (segment (start 102.620003 108.071853) (end 102.620003 114.986852) (width 0.4) (layer "F.Cu") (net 8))
 (segment (start 103.935004 106.756852) (end 102.620003 108.071853) (width 0.4) (layer "F.Cu") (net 8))
 (segment (start 102.620003 114.986852) (end 102.420003 115.186852) (width 0.4) (layer "F.Cu") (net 8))
 (segment (start 102.420003 115.186852) (end 102.420003 118.636852) (width 0.4) (layer "F.Cu") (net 8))
 (segment (start 107.600003 114.834352) (end 105.870003 114.834352) (width 0.4) (layer "F.Cu") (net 22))
 (segment (start 99.960003 111.836852) (end 98.730003 113.066852) (width 0.4) (layer "F.Cu") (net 22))
 (segment (start 98.730003 113.066852) (end 98.720003 113.066852) (width 0.4) (layer "F.Cu") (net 22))
 (via (at 105.870003 114.834352) (size 0.6) (drill 0.3) (layers "F.Cu" "B.Cu") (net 22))
 (via (at 98.720003 113.066852) (size 0.6) (drill 0.3) (layers "F.Cu" "B.Cu") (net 22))
 (segment (start 98.720003 113.066852) (end 100.487503 114.834352) (width 0.4) (layer "B.Cu") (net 22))
 (segment (start 117.070003 108.066852) (end 119.200003 110.196852) (width 0.4) (layer "B.Cu") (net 22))
 (segment (start 113.000003 116.396852) (end 107.432503 116.396852) (width 0.4) (layer "B.Cu") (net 22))
 (segment (start 119.200003 110.196852) (end 113.000003 116.396852) (width 0.4) (layer "B.Cu") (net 22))
 (segment (start 100.487503 114.834352) (end 105.870003 114.834352) (width 0.4) (layer "B.Cu") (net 22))
 (segment (start 107.432503 116.396852) (end 105.870003 114.834352) (width 0.4) (layer "B.Cu") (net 22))
 (segment (start 117.070003 107.996852) (end 117.070003 108.066852) (width 0.4) (layer "B.Cu") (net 22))
 (segment (start 95.83 94.908019) (end 95.83 94.92) (width 0.4) (layer "F.Cu") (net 6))
 (segment (start 97.421573 93.316446) (end 95.83 94.908019) (width 0.4) (layer "F.Cu") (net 6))
 (via (at 95.83 94.92) (size 0.6) (drill 0.3) (layers "F.Cu" "B.Cu") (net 6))
 (segment (start 94.580003 101.186852) (end 87.770003 107.996852) (width 0.4) (layer "B.Cu") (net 6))
 (segment (start 95.83 99.936855) (end 94.580003 101.186852) (width 0.4) (layer "B.Cu") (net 6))
 (segment (start 109.49 91.08) (end 109.49 91.126852) (width 0.4) (layer "B.Cu") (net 6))
 (segment (start 109.260003 91.086852) (end 109.483148 91.086852) (width 0.4) (layer "B.Cu") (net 6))
 (segment (start 95.83 94.92) (end 95.83 99.936855) (width 0.4) (layer "B.Cu") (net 6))
 (segment (start 109.483148 91.086852) (end 109.49 91.08) (width 0.4) (layer "B.Cu") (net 6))
 (segment (start 109.49 91.126852) (end 99.43 101.186852) (width 0.4) (layer "B.Cu") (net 6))
 (segment (start 99.43 101.186852) (end 94.580003 101.186852) (width 0.4) (layer "B.Cu") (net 6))
 (segment (start 102.220003 110.976852) (end 101.830003 110.586852) (width 0.4) (layer "B.Cu") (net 6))
 (segment (start 117.652896 109.453959) (end 116.030003 111.076852) (width 0.4) (layer "F.Cu") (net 13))
 (segment (start 87.24711 109.953959) (end 87.54711 109.953959) (width 0.4) (layer "F.Cu") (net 13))
 (segment (start 106.690003 104.226852) (end 104.920003 104.226852) (width 0.4) (layer "F.Cu") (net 13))
 (segment (start 87.54711 109.953959) (end 89.970003 112.376852) (width 0.4) (layer "F.Cu") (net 13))
 (segment (start 104.910003 104.216852) (end 104.910003 102.446852) (width 0.4) (layer "F.Cu") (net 13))
 (segment (start 104.920003 104.226852) (end 104.910003 104.216852) (width 0.4) (layer "F.Cu") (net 13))
 (segment (start 104.910003 102.446852) (end 104.930003 102.426852) (width 0.4) (layer "F.Cu") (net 13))
 (via (at 89.970003 112.376852) (size 0.6) (drill 0.3) (layers "F.Cu" "B.Cu") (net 13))
 (via (at 116.030003 111.076852) (size 0.6) (drill 0.3) (layers "F.Cu" "B.Cu") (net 13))
 (via (at 104.930003 102.426852) (size 0.6) (drill 0.3) (layers "F.Cu" "B.Cu") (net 13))
 (via (at 106.690003 104.226852) (size 0.6) (drill 0.3) (layers "F.Cu" "B.Cu") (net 13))
 (segment (start 99.920003 102.426852) (end 89.970003 112.376852) (width 0.4) (layer "B.Cu") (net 13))
 (segment (start 104.930003 98.176852) (end 104.930003 102.426852) (width 0.4) (layer "B.Cu") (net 13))
 (segment (start 104.930003 102.426852) (end 99.920003 102.426852) (width 0.4) (layer "B.Cu") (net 13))
 (segment (start 113.540003 111.076852) (end 106.690003 104.226852) (width 0.4) (layer "B.Cu") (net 13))
 (segment (start 116.030003 111.076852) (end 113.540003 111.076852) (width 0.4) (layer "B.Cu") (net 13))
 (segment (start 112.080003 91.026852) (end 104.930003 98.176852) (width 0.4) (layer "B.Cu") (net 13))
 (segment (start 107.250003 108.026852) (end 104.910003 108.026852) (width 0.4) (layer "F.Cu") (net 18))
 (segment (start 110.000003 105.276852) (end 107.250003 108.026852) (width 0.4) (layer "F.Cu") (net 18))
 (via (at 110.000003 105.276852) (size 0.6) (drill 0.3) (layers "F.Cu" "B.Cu") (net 18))
 (segment (start 110.000003 98.816852) (end 110.000003 105.276852) (width 0.4) (layer "B.Cu") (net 18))
 (segment (start 110.000003 95.636852) (end 110.000003 98.816852) (width 0.4) (layer "B.Cu") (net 18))
 (segment (start 114.630003 91.006852) (end 110.000003 95.636852) (width 0.4) (layer "B.Cu") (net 18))
 (segment (start 122.847919 94.606483) (end 106.88755 110.566852) (width 0.4) (layer "F.Cu") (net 3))
 (segment (start 106.88755 110.566852) (end 104.910003 110.566852) (width 0.4) (layer "F.Cu") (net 3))
 (segment (start 93.38 104.28) (end 93.443148 104.216852) (width 0.4) (layer "F.Cu") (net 17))
 (segment (start 112.479003 95.215852) (end 112.490003 95.226852) (width 0.4) (layer "F.Cu") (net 17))
 (segment (start 124.070003 106.146852) (end 124.070003 106.056852) (width 0.4) (layer "F.Cu") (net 17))
 (segment (start 87.18 98.08) (end 93.38 104.28) (width 0.4) (layer "F.Cu") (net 17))
 (segment (start 124.070003 101.046852) (end 121.160003 98.136852) (width 0.4) (layer "F.Cu") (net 17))
 (segment (start 87.18 96.39) (end 87.18 98.08) (width 0.4) (layer "F.Cu") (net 17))
 (segment (start 93.443148 104.216852) (end 99.960003 104.216852) (width 0.4) (layer "F.Cu") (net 17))
 (segment (start 108.982896 119.159745) (end 110.020003 120.196852) (width 0.4) (layer "F.Cu") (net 17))
 (segment (start 108.982896 119.133958) (end 108.982896 119.159745) (width 0.4) (layer "F.Cu") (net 17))
 (segment (start 108.961003 95.215852) (end 112.479003 95.215852) (width 0.4) (layer "F.Cu") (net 17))
 (segment (start 110.020003 120.196852) (end 124.070003 106.146852) (width 0.4) (layer "F.Cu") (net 17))
 (segment (start 99.960003 104.216852) (end 108.961003 95.215852) (width 0.4) (layer "F.Cu") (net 17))
 (segment (start 90.860003 91.936852) (end 90.860003 92.709997) (width 0.4) (layer "F.Cu") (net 17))
 (segment (start 124.070003 106.056852) (end 124.070003 101.046852) (width 0.4) (layer "F.Cu") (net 17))
 (segment (start 90.860003 92.709997) (end 87.18 96.39) (width 0.4) (layer "F.Cu") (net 17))
 (via (at 112.490003 95.226852) (size 0.6) (drill 0.3) (layers "F.Cu" "B.Cu") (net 17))
 (via (at 121.160003 98.136852) (size 0.6) (drill 0.3) (layers "F.Cu" "B.Cu") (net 17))
 (segment (start 119.760003 91.036852) (end 119.760003 96.736852) (width 0.4) (layer "B.Cu") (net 17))
 (segment (start 119.805003 96.781852) (end 121.160003 98.136852) (width 0.4) (layer "B.Cu") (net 17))
 (segment (start 118.250003 95.226852) (end 119.805003 96.781852) (width 0.4) (layer "B.Cu") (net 17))
 (segment (start 112.490003 95.226852) (end 118.250003 95.226852) (width 0.4) (layer "B.Cu") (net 17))
 (segment (start 119.760003 96.736852) (end 119.805003 96.781852) (width 0.4) (layer "B.Cu") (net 17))
 (segment (start 101.730003 114.38528) (end 96.724217 119.391066) (width 0.4) (layer "F.Cu") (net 19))
 (segment (start 114.390003 92.016852) (end 114.390003 97.776852) (width 0.4) (layer "F.Cu") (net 19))
 (segment (start 101.730003 107.616852) (end 101.730003 114.38528) (width 0.4) (layer "F.Cu") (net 19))
 (segment (start 114.390003 97.776852) (end 106.680003 105.486852) (width 0.4) (layer "F.Cu") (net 19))
 (segment (start 104.910003 105.486852) (end 103.860003 105.486852) (width 0.4) (layer "F.Cu") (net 19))
 (segment (start 106.680003 105.486852) (end 104.910003 105.486852) (width 0.4) (layer "F.Cu") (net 19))
 (segment (start 103.860003 105.486852) (end 101.730003 107.616852) (width 0.4) (layer "F.Cu") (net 19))
 (segment (start 87.130003 95.286852) (end 88.860003 93.556852) (width 0.4) (layer "F.Cu") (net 2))
 (segment (start 85.887726 95.286852) (end 87.130003 95.286852) (width 0.4) (layer "F.Cu") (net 2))
 (segment (start 83.510419 92.909545) (end 85.887726 95.286852) (width 0.4) (layer "F.Cu") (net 2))
 (segment (start 88.860003 93.556852) (end 88.860003 91.936852) (width 0.4) (layer "F.Cu") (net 2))
 (segment (start 84.629358 107.336207) (end 85.832896 108.539745) (width 0.4) (layer "F.Cu") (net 23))
 (segment (start 84.619359 107.336207) (end 84.629358 107.336207) (width 0.4) (layer "F.Cu") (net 23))
 (segment (start 94.114787 116.801636) (end 94.134787 116.801636) (width 0.4) (layer "F.Cu") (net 16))
 (segment (start 94.090003 116.756852) (end 95.310003 117.976852) (width 0.4) (layer "F.Cu") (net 16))
 (segment (start 110.39711 117.719746) (end 110.401893 117.719746) (width 0.4) (layer "F.Cu") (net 11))
 (segment (start 110.401893 117.719746) (end 111.620003 116.501636) (width 0.4) (layer "F.Cu") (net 11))
 (segment (start 116.390003 92.016852) (end 120.761718 92.016852) (width 0.4) (layer "F.Cu") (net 4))
 (segment (start 120.761718 92.016852) (end 121.672087 92.927221) (width 0.4) (layer "F.Cu") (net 4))
 (segment (start 102.420003 120.636852) (end 102.420003 122.369352) (width 0.4) (layer "F.Cu") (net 9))
 (segment (start 103.881003 113.20791) (end 103.881003 122.958352) (width 0.4) (layer "F.Cu") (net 12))
 (segment (start 103.300003 109.931853) (end 103.300003 112.62691) (width 0.4) (layer "F.Cu") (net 12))
 (segment (start 104.910003 109.296852) (end 103.935004 109.296852) (width 0.4) (layer "F.Cu") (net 12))
 (segment (start 103.300003 112.62691) (end 103.881003 113.20791) (width 0.4) (layer "F.Cu") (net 12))
 (segment (start 103.935004 109.296852) (end 103.300003 109.931853) (width 0.4) (layer "F.Cu") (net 12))
 (segment (start 103.881003 122.958352) (end 102.420003 124.419352) (width 0.4) (layer "F.Cu") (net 12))
 (segment (start 107.46 94.3) (end 102.83 98.93) (width 0.4) (layer "F.Cu") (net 5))
 (segment (start 107.600003 111.846855) (end 107.59 111.836852) (width 0.4) (layer "F.Cu") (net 5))
 (segment (start 112.42 94.3) (end 107.46 94.3) (width 0.4) (layer "F.Cu") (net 5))
 (segment (start 107.59 111.836852) (end 109.093148 111.836852) (width 0.4) (layer "F.Cu") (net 5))
 (segment (start 104.910003 111.836852) (end 107.59 111.836852) (width 0.4) (layer "F.Cu") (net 5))
 (segment (start 99.542894 97.382894) (end 99.542894 95.437766) (width 0.4) (layer "F.Cu") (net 5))
 (segment (start 107.600003 112.759352) (end 107.600003 111.846855) (width 0.4) (layer "F.Cu") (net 5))
 (segment (start 109.093148 111.836852) (end 113.08 107.85) (width 0.4) (layer "F.Cu") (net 5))
 (segment (start 101.09 98.93) (end 99.542894 97.382894) (width 0.4) (layer "F.Cu") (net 5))
 (segment (start 102.83 98.93) (end 101.09 98.93) (width 0.4) (layer "F.Cu") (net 5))
 (via (at 112.42 94.3) (size 0.6) (drill 0.3) (layers "F.Cu" "B.Cu") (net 5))
 (via (at 113.08 107.85) (size 0.6) (drill 0.3) (layers "F.Cu" "B.Cu") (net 5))
 (segment (start 112.42 94.3) (end 111.03 95.69) (width 0.4) (layer "B.Cu") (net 5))
 (segment (start 111.03 95.69) (end 111.03 104.24) (width 0.4) (layer "B.Cu") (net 5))
 (segment (start 111.03 104.24) (end 111.03 105.8) (width 0.4) (layer "B.Cu") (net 5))
 (segment (start 111.03 105.8) (end 113.08 107.85) (width 0.4) (layer "B.Cu") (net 5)))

